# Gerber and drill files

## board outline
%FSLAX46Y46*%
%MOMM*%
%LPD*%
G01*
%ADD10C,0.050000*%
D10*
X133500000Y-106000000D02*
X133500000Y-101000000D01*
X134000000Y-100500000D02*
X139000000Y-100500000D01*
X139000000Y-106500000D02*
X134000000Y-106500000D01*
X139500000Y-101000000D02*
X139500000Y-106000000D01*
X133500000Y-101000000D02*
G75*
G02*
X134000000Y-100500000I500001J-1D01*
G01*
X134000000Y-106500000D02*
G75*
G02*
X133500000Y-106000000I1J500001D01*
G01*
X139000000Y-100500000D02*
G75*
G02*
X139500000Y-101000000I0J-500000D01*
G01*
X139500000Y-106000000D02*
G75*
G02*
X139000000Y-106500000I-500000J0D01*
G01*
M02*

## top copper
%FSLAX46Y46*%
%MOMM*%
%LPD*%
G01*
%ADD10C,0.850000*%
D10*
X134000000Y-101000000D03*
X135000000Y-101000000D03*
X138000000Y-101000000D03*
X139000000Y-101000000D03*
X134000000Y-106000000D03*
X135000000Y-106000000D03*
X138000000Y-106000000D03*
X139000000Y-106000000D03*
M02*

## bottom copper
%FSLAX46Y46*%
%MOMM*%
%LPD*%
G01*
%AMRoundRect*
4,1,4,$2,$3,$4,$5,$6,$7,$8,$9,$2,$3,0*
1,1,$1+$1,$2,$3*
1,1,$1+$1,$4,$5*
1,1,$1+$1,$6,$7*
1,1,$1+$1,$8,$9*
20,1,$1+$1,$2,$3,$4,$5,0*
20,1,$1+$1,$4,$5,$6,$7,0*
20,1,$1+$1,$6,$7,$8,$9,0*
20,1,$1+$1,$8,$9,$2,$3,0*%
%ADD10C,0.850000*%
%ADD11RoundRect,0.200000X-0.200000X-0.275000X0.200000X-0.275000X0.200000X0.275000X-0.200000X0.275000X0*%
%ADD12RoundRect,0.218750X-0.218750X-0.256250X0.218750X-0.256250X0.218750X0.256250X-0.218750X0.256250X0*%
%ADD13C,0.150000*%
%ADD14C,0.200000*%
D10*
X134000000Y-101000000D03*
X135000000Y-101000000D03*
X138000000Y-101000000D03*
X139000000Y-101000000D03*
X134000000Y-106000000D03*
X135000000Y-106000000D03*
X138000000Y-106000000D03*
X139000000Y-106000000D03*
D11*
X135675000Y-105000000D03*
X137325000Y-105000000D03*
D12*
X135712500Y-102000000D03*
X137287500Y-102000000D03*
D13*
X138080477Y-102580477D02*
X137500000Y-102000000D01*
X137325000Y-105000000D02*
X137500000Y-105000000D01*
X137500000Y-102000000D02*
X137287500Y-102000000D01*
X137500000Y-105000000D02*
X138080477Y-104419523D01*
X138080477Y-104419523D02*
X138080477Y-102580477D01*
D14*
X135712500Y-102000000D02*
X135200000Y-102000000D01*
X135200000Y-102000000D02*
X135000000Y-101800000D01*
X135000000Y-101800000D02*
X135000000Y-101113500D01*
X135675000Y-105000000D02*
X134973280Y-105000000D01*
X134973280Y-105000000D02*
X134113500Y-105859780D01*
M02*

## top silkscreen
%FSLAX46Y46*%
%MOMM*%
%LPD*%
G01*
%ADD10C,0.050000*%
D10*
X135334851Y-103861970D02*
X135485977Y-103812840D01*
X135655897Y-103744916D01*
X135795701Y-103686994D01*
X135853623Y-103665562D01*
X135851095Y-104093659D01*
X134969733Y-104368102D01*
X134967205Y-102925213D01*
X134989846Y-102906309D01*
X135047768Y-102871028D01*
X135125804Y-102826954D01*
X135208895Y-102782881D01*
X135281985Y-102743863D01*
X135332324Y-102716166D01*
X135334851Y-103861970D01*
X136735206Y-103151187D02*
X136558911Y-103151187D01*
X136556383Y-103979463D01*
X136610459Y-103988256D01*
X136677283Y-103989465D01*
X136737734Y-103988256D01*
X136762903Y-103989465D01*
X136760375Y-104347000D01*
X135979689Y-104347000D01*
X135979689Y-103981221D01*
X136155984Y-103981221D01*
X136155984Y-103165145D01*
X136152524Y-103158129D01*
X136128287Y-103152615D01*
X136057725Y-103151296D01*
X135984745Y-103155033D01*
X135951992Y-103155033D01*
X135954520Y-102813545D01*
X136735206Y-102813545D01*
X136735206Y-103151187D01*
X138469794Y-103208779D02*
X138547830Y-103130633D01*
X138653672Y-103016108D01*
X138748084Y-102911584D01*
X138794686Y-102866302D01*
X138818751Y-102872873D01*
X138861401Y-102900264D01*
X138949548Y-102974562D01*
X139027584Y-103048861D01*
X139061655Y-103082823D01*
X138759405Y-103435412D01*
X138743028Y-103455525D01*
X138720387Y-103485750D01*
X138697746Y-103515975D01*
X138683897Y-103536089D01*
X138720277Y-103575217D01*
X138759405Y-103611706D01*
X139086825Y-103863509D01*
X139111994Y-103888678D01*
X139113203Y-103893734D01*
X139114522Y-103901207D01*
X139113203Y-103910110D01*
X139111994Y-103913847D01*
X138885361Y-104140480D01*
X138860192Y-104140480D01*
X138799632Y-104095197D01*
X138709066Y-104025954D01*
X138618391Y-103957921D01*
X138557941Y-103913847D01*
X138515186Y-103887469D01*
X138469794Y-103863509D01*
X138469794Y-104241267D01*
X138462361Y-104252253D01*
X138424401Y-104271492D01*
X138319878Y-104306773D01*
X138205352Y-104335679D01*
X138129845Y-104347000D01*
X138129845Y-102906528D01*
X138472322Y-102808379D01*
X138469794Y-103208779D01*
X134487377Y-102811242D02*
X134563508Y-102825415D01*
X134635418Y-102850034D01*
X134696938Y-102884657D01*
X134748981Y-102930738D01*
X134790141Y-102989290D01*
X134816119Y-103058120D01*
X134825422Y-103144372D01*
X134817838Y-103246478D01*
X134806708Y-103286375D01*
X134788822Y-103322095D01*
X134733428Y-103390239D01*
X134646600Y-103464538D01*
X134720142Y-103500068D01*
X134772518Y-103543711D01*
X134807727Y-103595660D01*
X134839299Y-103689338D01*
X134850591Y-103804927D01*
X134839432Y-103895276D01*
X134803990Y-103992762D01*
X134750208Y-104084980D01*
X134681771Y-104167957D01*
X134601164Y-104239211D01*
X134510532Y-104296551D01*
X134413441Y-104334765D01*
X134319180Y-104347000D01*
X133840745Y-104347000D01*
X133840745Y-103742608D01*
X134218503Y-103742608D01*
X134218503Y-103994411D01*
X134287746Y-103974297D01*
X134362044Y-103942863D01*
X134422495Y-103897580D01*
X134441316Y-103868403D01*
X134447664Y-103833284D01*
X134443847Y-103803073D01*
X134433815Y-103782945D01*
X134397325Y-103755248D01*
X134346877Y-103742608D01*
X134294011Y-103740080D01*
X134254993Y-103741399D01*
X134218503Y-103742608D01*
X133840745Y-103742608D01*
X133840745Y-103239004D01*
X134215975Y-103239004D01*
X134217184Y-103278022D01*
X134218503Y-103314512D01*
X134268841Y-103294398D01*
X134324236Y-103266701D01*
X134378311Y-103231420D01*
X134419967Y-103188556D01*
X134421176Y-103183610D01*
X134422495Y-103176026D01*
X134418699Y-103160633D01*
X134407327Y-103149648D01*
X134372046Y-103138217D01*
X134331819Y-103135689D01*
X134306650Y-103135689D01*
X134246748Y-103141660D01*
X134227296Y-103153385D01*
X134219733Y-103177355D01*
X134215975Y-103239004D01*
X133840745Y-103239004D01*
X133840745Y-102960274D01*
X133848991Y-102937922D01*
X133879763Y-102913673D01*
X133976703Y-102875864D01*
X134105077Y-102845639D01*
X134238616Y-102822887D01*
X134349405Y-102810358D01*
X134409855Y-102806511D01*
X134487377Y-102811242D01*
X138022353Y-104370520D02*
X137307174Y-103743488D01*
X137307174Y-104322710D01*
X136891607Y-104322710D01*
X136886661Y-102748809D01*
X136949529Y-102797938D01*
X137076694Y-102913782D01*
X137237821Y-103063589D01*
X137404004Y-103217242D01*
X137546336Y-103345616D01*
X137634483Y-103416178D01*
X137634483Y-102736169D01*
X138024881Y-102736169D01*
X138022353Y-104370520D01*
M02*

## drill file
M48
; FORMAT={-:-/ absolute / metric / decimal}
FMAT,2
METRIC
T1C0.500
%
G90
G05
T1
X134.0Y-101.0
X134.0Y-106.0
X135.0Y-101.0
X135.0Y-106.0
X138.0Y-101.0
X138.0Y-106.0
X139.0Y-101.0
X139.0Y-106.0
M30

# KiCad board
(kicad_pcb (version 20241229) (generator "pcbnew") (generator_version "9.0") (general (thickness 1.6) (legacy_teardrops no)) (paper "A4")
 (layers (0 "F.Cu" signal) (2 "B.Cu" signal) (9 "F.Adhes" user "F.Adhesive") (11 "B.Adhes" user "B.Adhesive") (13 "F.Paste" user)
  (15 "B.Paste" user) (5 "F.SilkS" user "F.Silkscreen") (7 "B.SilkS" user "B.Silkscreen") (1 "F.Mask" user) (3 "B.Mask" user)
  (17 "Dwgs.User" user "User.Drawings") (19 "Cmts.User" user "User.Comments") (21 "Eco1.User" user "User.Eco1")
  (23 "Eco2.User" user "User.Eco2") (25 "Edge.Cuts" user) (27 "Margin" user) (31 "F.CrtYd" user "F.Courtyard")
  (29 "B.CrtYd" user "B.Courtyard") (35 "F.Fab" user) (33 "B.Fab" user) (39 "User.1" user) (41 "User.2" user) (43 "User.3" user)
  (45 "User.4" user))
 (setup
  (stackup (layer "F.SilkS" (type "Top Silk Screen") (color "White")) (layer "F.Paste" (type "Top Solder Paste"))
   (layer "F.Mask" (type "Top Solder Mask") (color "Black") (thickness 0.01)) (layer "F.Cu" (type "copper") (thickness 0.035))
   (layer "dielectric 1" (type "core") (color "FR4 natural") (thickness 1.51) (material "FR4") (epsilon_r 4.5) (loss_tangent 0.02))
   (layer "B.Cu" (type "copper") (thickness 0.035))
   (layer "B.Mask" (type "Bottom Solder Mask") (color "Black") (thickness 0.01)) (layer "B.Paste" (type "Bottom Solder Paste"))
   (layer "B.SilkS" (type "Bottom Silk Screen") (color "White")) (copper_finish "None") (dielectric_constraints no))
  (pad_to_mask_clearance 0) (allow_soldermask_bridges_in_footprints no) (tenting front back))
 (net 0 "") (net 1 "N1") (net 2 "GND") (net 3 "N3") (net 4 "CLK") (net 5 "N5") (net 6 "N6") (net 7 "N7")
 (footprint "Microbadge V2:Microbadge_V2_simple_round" (layer "F.Cu") (at 136.5 103.5)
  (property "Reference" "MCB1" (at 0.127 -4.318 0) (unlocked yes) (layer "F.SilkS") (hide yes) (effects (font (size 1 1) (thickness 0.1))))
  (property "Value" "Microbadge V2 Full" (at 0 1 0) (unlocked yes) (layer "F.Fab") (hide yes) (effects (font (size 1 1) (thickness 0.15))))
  (fp_line (start -3 2.5) (end -3 -2.5) (stroke (width 0.05) (type default)) (layer "Edge.Cuts"))
  (fp_line (start -2.5 -3) (end 2.5 -3) (stroke (width 0.05) (type default)) (layer "Edge.Cuts"))
  (fp_line (start 2.5 3) (end -2.5 3) (stroke (width 0.05) (type default)) (layer "Edge.Cuts"))
  (fp_line (start 3 -2.5) (end 3 2.5) (stroke (width 0.05) (type default)) (layer "Edge.Cuts"))
  (fp_arc (start -3 -2.5) (mid -2.853553 -2.853553) (end -2.5 -3) (stroke (width 0.05) (type default)) (layer "Edge.Cuts"))
  (fp_arc (start -2.5 3) (mid -2.853553 2.853553) (end -3 2.5) (stroke (width 0.05) (type default)) (layer "Edge.Cuts"))
  (fp_arc (start 2.5 -3) (mid 2.853553 -2.853553) (end 3 -2.5) (stroke (width 0.05) (type default)) (layer "Edge.Cuts"))
  (fp_arc (start 3 2.5) (mid 2.853553 2.853553) (end 2.5 3) (stroke (width 0.05) (type default)) (layer "Edge.Cuts"))
  (pad "1" thru_hole circle (at -2.5 -2.5 90) (size 0.85 0.85) (drill 0.5) (layers "*.Cu" "*.Mask") (remove_unused_layers no) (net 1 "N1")
   (thermal_bridge_angle 90))
  (pad "2" thru_hole circle (at -1.5 -2.5 90) (size 0.85 0.85) (drill 0.5) (layers "*.Cu" "*.Mask") (remove_unused_layers no) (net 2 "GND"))
  (pad "5" thru_hole circle (at 1.5 -2.5 90) (size 0.85 0.85) (drill 0.5) (layers "*.Cu" "*.Mask") (remove_unused_layers no) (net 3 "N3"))
  (pad "6" thru_hole circle (at 2.5 -2.5 90) (size 0.85 0.85) (drill 0.5) (layers "*.Cu" "*.Mask") (remove_unused_layers no) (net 2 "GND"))
  (pad "7" thru_hole circle (at -2.5 2.5 90) (size 0.85 0.85) (drill 0.5) (layers "*.Cu" "*.Mask") (remove_unused_layers no) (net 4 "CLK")
   (thermal_bridge_angle 90))
  (pad "8" thru_hole circle (at -1.5 2.5 90) (size 0.85 0.85) (drill 0.5) (layers "*.Cu" "*.Mask") (remove_unused_layers no) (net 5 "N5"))
  (pad "11" thru_hole circle (at 1.5 2.5 90) (size 0.85 0.85) (drill 0.5) (layers "*.Cu" "*.Mask") (remove_unused_layers no) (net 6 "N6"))
  (pad "12" thru_hole circle (at 2.5 2.5 90) (size 0.85 0.85) (drill 0.5) (layers "*.Cu" "*.Mask") (remove_unused_layers no) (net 2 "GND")))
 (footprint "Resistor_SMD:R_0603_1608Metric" (layer "B.Cu") (at 136.5 105)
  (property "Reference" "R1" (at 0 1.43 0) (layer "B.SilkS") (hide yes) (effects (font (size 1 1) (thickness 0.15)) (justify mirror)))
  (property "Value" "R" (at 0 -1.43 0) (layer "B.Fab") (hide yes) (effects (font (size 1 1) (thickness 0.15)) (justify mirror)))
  (pad "1" smd roundrect (at -0.825 0) (size 0.8 0.95) (layers "B.Cu" "B.Mask" "B.Paste") (roundrect_rratio 0.25) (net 4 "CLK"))
  (pad "2" smd roundrect (at 0.825 0) (size 0.8 0.95) (layers "B.Cu" "B.Mask" "B.Paste") (roundrect_rratio 0.25) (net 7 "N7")))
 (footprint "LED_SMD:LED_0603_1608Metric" (layer "B.Cu") (at 136.5 102)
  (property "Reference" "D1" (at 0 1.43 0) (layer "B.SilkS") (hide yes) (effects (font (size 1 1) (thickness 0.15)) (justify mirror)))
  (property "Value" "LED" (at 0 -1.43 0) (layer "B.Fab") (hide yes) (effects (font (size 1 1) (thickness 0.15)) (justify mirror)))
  (pad "1" smd roundrect (at -0.7875 0) (size 0.875 0.95) (layers "B.Cu" "B.Mask" "B.Paste") (roundrect_rratio 0.25) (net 2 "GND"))
  (pad "2" smd roundrect (at 0.7875 0) (size 0.875 0.95) (layers "B.Cu" "B.Mask" "B.Paste") (roundrect_rratio 0.25) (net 7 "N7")))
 (gr_poly
  (pts (xy 135.334851 103.86197) (xy 135.485977 103.81284) (xy 135.655897 103.744916) (xy 135.795701 103.686994) (xy 135.853623 103.665562)
   (xy 135.851095 104.093659) (xy 134.969733 104.368102) (xy 134.967205 102.925213) (xy 134.989846 102.906309) (xy 135.047768 102.871028)
   (xy 135.125804 102.826954) (xy 135.208895 102.782881) (xy 135.281985 102.743863) (xy 135.332324 102.716166))
  (stroke (width 0.05) (type solid)) (fill no) (layer "F.SilkS"))
 (gr_poly
  (pts (xy 136.735206 103.151187) (xy 136.558911 103.151187) (xy 136.556383 103.979463) (xy 136.610459 103.988256)
   (xy 136.677283 103.989465) (xy 136.737734 103.988256) (xy 136.762903 103.989465) (xy 136.760375 104.347) (xy 135.979689 104.347)
   (xy 135.979689 103.981221) (xy 136.155984 103.981221) (xy 136.155984 103.165145) (xy 136.152524 103.158129) (xy 136.128287 103.152615)
   (xy 136.057725 103.151296) (xy 135.984745 103.155033) (xy 135.951992 103.155033) (xy 135.95452 102.813545) (xy 136.735206 102.813545))
  (stroke (width 0.05) (type solid)) (fill no) (layer "F.SilkS"))
 (gr_poly
  (pts (xy 138.469794 103.208779) (xy 138.54783 103.130633) (xy 138.653672 103.016108) (xy 138.748084 102.911584) (xy 138.794686 102.866302)
   (xy 138.818751 102.872873) (xy 138.861401 102.900264) (xy 138.949548 102.974562) (xy 139.027584 103.048861) (xy 139.061655 103.082823)
   (xy 138.759405 103.435412) (xy 138.743028 103.455525) (xy 138.720387 103.48575) (xy 138.697746 103.515975) (xy 138.683897 103.536089)
   (xy 138.720277 103.575217) (xy 138.759405 103.611706) (xy 139.086825 103.863509) (xy 139.111994 103.888678) (xy 139.113203 103.893734)
   (xy 139.114522 103.901207) (xy 139.113203 103.91011) (xy 139.111994 103.913847) (xy 138.885361 104.14048) (xy 138.860192 104.14048)
   (xy 138.799632 104.095197) (xy 138.709066 104.025954) (xy 138.618391 103.957921) (xy 138.557941 103.913847) (xy 138.515186 103.887469)
   (xy 138.469794 103.863509) (xy 138.469794 104.241267) (xy 138.462361 104.252253) (xy 138.424401 104.271492) (xy 138.319878 104.306773)
   (xy 138.205352 104.335679) (xy 138.129845 104.347) (xy 138.129845 102.906528) (xy 138.472322 102.808379))
  (stroke (width 0.05) (type solid)) (fill no) (layer "F.SilkS"))
 (gr_poly
  (pts (xy 134.487377 102.811242) (xy 134.563508 102.825415) (xy 134.635418 102.850034) (xy 134.696938 102.884657)
   (xy 134.748981 102.930738) (xy 134.790141 102.98929) (xy 134.816119 103.05812) (xy 134.825422 103.144372) (xy 134.817838 103.246478)
   (xy 134.806708 103.286375) (xy 134.788822 103.322095) (xy 134.733428 103.390239) (xy 134.6466 103.464538) (xy 134.720142 103.500068)
   (xy 134.772518 103.543711) (xy 134.807727 103.59566) (xy 134.839299 103.689338) (xy 134.850591 103.804927) (xy 134.839432 103.895276)
   (xy 134.80399 103.992762) (xy 134.750208 104.08498) (xy 134.681771 104.167957) (xy 134.601164 104.239211) (xy 134.510532 104.296551)
   (xy 134.413441 104.334765) (xy 134.31918 104.347) (xy 133.840745 104.347) (xy 133.840745 103.742608) (xy 134.218503 103.742608)
   (xy 134.218503 103.994411) (xy 134.287746 103.974297) (xy 134.362044 103.942863) (xy 134.422495 103.89758) (xy 134.441316 103.868403)
   (xy 134.447664 103.833284) (xy 134.443847 103.803073) (xy 134.433815 103.782945) (xy 134.397325 103.755248) (xy 134.346877 103.742608)
   (xy 134.294011 103.74008) (xy 134.254993 103.741399) (xy 134.218503 103.742608) (xy 133.840745 103.742608) (xy 133.840745 103.239004)
   (xy 134.215975 103.239004) (xy 134.217184 103.278022) (xy 134.218503 103.314512) (xy 134.268841 103.294398) (xy 134.324236 103.266701)
   (xy 134.378311 103.23142) (xy 134.419967 103.188556) (xy 134.421176 103.18361) (xy 134.422495 103.176026) (xy 134.418699 103.160633)
   (xy 134.407327 103.149648) (xy 134.372046 103.138217) (xy 134.331819 103.135689) (xy 134.30665 103.135689) (xy 134.246748 103.14166)
   (xy 134.227296 103.153385) (xy 134.219733 103.177355) (xy 134.215975 103.239004) (xy 133.840745 103.239004) (xy 133.840745 102.960274)
   (xy 133.848991 102.937922) (xy 133.879763 102.913673) (xy 133.976703 102.875864) (xy 134.105077 102.845639) (xy 134.238616 102.822887)
   (xy 134.349405 102.810358) (xy 134.409855 102.806511))
  (stroke (width 0.05) (type solid)) (fill no) (layer "F.SilkS"))
 (gr_poly
  (pts (xy 138.022353 104.37052) (xy 137.307174 103.743488) (xy 137.307174 104.32271) (xy 136.891607 104.32271) (xy 136.886661 102.748809)
   (xy 136.949529 102.797938) (xy 137.076694 102.913782) (xy 137.237821 103.063589) (xy 137.404004 103.217242) (xy 137.546336 103.345616)
   (xy 137.634483 103.416178) (xy 137.634483 102.736169) (xy 138.024881 102.736169))
  (stroke (width 0.05) (type solid)) (fill no) (layer "F.SilkS"))
 (segment (start 138.080477 102.580477) (end 137.5 102) (width 0.15) (layer "B.Cu") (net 7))
 (segment (start 137.325 105) (end 137.5 105) (width 0.15) (layer "B.Cu") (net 7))
 (segment (start 137.5 102) (end 137.2875 102) (width 0.15) (layer "B.Cu") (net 7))
 (segment (start 137.5 105) (end 138.080477 104.419523) (width 0.15) (layer "B.Cu") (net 7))
 (segment (start 138.080477 104.419523) (end 138.080477 102.580477) (width 0.15) (layer "B.Cu") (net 7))
 (segment (start 135.7125 102) (end 135.2 102) (width 0.2) (layer "B.Cu") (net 2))
 (segment (start 135.2 102) (end 135 101.8) (width 0.2) (layer "B.Cu") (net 2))
 (segment (start 135 101.8) (end 135 101.1135) (width 0.2) (layer "B.Cu") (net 2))
 (segment (start 135.675 105) (end 134.97328 105) (width 0.2) (layer "B.Cu") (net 4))
 (segment (start 134.97328 105) (end 134.1135 105.85978) (width 0.2) (layer "B.Cu") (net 4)))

